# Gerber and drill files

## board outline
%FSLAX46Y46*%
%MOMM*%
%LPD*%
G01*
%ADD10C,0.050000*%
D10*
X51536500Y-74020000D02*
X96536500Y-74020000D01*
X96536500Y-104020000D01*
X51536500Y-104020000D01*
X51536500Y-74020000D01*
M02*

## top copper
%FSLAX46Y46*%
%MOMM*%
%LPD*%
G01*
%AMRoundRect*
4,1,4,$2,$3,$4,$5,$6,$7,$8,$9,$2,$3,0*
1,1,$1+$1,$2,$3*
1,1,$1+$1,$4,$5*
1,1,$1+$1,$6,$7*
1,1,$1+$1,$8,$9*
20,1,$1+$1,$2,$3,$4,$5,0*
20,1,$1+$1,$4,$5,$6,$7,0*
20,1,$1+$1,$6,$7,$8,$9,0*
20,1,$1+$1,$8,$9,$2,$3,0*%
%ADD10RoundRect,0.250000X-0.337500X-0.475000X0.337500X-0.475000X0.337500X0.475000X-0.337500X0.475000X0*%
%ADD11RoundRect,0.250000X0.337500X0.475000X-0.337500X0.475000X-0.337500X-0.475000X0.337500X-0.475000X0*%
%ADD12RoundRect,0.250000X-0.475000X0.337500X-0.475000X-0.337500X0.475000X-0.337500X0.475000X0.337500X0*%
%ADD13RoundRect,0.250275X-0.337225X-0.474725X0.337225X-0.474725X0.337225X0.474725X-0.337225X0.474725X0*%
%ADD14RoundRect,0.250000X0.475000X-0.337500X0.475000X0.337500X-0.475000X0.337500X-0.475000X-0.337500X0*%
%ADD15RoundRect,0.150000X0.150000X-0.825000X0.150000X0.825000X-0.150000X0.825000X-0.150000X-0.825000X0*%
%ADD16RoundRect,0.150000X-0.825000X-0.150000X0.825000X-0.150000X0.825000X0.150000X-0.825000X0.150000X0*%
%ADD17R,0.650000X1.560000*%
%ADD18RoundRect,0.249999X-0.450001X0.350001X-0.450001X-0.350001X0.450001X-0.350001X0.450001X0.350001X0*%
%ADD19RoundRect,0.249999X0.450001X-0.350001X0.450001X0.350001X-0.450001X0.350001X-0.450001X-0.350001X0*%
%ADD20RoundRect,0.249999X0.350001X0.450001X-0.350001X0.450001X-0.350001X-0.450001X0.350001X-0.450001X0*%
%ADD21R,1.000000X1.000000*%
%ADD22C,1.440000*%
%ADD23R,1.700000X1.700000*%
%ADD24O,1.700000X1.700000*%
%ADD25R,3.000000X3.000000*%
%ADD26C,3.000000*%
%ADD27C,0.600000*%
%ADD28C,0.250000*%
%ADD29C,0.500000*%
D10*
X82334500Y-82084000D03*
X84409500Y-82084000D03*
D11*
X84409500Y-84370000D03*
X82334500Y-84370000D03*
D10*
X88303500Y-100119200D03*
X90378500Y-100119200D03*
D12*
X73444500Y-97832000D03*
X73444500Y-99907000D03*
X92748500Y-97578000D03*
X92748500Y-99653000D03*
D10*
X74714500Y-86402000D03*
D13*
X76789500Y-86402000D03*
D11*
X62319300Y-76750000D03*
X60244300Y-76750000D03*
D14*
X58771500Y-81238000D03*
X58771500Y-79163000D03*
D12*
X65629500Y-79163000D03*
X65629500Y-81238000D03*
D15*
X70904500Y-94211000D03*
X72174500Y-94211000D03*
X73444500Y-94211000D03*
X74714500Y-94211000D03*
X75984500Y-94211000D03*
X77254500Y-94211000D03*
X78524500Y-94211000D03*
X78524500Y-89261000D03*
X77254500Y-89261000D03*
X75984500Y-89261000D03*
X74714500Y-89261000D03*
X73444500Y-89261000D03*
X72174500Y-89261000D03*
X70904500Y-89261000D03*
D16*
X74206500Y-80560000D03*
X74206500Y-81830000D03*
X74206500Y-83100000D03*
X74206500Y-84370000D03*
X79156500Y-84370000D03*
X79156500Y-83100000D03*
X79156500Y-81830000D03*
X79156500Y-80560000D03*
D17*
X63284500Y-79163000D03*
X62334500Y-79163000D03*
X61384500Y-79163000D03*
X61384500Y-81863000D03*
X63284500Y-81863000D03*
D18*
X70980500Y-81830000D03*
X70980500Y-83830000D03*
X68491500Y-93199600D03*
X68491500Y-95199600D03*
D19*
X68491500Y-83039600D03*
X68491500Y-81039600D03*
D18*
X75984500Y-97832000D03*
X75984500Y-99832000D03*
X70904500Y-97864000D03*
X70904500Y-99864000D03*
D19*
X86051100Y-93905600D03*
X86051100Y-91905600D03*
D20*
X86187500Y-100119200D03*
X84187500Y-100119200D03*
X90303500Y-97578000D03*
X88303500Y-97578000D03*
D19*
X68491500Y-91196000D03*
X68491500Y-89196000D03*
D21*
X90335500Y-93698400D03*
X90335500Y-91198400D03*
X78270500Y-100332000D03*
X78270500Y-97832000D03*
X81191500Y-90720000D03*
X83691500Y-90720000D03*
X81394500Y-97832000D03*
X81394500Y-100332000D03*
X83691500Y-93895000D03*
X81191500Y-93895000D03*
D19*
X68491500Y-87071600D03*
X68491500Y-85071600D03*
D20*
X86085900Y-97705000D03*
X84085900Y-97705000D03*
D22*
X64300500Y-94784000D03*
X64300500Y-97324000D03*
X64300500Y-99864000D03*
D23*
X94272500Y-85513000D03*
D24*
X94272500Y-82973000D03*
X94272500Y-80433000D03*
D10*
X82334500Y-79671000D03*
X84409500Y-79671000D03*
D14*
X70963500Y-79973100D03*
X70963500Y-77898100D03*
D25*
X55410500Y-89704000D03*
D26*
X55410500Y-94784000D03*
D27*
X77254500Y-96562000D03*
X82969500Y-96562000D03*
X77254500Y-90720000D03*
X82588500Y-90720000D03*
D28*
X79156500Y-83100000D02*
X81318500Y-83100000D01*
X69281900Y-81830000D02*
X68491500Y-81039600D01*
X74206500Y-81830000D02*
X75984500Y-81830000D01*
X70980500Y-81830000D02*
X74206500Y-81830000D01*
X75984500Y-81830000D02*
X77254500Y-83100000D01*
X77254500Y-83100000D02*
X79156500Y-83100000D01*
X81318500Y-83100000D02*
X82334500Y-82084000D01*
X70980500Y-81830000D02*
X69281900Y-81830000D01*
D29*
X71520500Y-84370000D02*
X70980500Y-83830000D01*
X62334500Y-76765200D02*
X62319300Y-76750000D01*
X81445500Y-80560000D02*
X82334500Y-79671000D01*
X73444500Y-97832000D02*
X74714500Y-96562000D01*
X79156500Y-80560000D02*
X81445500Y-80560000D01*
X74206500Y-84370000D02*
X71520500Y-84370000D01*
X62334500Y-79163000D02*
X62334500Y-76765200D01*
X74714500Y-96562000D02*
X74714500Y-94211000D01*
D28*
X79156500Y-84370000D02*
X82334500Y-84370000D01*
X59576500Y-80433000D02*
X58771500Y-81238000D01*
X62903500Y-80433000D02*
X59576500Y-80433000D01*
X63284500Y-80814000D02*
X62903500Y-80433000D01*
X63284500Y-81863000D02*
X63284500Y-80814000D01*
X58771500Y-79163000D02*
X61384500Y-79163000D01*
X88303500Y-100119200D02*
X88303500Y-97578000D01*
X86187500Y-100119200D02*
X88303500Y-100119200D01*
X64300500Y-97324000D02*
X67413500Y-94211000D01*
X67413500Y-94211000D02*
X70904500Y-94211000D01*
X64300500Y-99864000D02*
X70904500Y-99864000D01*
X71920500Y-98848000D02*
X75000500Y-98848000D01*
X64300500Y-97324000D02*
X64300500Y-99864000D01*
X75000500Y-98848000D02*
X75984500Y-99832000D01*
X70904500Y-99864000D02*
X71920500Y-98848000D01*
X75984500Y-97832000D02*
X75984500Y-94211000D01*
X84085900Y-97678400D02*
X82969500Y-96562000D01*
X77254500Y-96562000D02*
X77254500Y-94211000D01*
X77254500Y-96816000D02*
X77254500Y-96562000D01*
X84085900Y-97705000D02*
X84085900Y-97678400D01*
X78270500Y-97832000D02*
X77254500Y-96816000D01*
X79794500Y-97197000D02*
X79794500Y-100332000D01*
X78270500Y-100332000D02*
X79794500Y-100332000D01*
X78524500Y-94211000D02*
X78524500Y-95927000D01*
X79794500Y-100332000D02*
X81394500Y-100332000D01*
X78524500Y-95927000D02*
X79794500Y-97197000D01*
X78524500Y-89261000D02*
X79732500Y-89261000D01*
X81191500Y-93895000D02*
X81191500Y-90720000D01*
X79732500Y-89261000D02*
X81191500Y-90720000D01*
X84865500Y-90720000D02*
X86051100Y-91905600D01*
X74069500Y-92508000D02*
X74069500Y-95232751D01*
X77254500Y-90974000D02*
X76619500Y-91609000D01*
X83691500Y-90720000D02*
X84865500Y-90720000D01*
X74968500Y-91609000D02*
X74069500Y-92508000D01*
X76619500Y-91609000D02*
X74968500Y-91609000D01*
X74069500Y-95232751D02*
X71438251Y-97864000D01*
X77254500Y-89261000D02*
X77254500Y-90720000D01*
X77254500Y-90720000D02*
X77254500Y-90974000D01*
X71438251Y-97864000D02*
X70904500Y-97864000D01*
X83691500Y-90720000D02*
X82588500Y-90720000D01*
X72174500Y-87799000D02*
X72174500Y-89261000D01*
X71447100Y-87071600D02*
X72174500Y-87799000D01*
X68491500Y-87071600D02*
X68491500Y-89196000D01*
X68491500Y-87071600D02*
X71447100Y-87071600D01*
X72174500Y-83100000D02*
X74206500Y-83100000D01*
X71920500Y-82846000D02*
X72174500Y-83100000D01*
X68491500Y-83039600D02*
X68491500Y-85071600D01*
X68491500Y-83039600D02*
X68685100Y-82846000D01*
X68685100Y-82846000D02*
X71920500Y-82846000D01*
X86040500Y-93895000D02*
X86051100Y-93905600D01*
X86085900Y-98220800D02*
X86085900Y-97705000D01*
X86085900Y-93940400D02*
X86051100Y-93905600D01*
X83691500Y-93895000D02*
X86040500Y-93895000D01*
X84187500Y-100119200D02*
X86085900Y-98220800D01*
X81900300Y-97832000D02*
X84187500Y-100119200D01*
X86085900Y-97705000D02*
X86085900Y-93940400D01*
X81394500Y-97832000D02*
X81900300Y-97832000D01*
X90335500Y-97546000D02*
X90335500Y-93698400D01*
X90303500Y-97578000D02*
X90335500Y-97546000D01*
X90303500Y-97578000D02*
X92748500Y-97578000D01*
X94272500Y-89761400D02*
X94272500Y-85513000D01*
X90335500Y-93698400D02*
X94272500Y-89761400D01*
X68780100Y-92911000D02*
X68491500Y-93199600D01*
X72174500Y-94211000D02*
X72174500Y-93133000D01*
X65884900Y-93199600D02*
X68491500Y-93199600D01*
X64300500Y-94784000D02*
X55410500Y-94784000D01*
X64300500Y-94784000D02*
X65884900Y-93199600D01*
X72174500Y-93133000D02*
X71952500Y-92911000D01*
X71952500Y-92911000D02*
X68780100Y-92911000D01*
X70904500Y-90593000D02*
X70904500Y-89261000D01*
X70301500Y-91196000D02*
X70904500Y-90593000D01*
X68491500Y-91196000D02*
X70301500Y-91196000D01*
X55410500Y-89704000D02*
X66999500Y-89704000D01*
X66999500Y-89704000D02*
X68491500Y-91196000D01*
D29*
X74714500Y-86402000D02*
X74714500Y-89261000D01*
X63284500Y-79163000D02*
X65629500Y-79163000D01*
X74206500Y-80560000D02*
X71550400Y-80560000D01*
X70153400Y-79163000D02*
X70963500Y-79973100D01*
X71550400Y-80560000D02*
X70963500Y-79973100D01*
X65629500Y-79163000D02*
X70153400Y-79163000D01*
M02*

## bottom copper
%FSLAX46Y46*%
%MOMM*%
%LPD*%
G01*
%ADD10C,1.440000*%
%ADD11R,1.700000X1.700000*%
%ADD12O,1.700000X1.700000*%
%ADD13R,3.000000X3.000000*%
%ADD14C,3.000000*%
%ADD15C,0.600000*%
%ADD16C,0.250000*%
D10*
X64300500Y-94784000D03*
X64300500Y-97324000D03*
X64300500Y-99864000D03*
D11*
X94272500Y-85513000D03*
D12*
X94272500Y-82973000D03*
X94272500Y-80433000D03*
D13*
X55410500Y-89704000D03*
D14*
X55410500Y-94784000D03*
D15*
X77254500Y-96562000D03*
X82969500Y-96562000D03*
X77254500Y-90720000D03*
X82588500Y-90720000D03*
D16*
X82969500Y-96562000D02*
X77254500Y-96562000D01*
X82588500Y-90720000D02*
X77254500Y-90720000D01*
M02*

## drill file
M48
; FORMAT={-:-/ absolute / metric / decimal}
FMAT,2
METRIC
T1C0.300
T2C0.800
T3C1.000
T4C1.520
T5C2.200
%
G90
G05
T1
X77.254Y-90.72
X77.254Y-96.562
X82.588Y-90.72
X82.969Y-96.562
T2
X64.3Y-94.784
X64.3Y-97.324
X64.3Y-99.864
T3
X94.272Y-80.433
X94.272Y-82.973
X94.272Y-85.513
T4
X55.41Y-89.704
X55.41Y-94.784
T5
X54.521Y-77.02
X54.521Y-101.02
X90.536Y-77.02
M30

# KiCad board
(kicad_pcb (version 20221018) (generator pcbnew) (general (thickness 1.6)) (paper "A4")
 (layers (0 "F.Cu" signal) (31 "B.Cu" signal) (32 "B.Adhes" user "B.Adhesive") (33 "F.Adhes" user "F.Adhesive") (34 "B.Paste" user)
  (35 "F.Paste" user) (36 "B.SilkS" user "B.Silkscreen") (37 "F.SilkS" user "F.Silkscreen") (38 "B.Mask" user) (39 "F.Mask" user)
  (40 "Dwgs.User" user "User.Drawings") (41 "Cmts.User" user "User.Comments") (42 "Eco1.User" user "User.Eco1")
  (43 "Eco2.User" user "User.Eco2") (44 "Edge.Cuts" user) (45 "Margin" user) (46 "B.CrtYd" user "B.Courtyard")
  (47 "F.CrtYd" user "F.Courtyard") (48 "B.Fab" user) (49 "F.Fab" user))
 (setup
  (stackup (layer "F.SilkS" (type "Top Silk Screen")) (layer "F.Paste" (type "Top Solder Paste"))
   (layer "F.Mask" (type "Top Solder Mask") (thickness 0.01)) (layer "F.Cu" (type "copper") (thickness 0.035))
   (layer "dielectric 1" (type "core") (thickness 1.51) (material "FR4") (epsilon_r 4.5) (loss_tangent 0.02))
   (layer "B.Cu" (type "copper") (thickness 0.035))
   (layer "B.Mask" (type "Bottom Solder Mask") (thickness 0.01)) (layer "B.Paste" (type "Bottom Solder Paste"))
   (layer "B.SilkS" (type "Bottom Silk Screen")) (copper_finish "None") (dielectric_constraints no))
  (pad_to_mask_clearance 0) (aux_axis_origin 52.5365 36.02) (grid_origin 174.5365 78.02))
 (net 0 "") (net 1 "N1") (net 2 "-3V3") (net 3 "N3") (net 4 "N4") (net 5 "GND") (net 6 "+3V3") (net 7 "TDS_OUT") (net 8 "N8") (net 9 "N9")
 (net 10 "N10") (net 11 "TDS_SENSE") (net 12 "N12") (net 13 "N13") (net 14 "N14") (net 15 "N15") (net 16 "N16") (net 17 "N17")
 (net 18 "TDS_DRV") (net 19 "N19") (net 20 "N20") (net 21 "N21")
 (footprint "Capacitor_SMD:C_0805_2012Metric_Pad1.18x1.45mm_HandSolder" (layer "F.Cu") (at 83.372 82.084)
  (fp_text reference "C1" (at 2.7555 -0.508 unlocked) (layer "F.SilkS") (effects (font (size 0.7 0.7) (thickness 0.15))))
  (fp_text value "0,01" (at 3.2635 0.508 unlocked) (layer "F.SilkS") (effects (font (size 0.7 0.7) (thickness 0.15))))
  (pad "1" smd roundrect (at -1.0375 0) (size 1.175 1.45) (layers "F.Cu" "F.Paste" "F.Mask") (roundrect_rratio 0.2127659574) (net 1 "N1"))
  (pad "2" smd roundrect (at 1.0375 0) (size 1.175 1.45) (layers "F.Cu" "F.Paste" "F.Mask") (roundrect_rratio 0.2127659574) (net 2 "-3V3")))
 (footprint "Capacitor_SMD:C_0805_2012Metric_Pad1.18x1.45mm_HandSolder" (layer "F.Cu") (at 83.372 84.37 180)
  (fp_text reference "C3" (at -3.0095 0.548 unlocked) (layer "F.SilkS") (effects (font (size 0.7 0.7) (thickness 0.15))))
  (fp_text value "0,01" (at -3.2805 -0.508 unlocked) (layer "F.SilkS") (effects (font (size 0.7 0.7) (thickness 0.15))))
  (pad "1" smd roundrect (at -1.0375 0 180) (size 1.175 1.45) (layers "F.Cu" "F.Paste" "F.Mask") (roundrect_rratio 0.2127659574)
   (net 2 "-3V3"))
  (pad "2" smd roundrect (at 1.0375 0 180) (size 1.175 1.45) (layers "F.Cu" "F.Paste" "F.Mask") (roundrect_rratio 0.2127659574) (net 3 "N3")))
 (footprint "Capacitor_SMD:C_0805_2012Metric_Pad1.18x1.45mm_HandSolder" (layer "F.Cu") (at 89.341 100.1192)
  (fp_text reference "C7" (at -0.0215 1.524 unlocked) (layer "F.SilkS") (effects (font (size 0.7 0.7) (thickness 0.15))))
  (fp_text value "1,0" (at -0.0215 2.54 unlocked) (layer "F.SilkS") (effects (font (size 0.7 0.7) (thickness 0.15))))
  (pad "1" smd roundrect (at -1.0375 0) (size 1.175 1.45) (layers "F.Cu" "F.Paste" "F.Mask") (roundrect_rratio 0.2127659574) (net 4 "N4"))
  (pad "2" smd roundrect (at 1.0375 0) (size 1.175 1.45) (layers "F.Cu" "F.Paste" "F.Mask") (roundrect_rratio 0.2127659574) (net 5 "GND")))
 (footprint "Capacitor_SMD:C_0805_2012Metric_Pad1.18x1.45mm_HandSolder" (layer "F.Cu") (at 73.4445 98.8695 -90)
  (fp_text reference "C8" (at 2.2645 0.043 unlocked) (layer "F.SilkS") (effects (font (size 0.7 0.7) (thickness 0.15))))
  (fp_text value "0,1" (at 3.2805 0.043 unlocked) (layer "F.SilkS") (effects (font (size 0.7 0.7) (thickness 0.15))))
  (pad "1" smd roundrect (at -1.0375 0 270) (size 1.175 1.45) (layers "F.Cu" "F.Paste" "F.Mask") (roundrect_rratio 0.2127659574)
   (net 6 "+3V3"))
  (pad "2" smd roundrect (at 1.0375 0 270) (size 1.175 1.45) (layers "F.Cu" "F.Paste" "F.Mask") (roundrect_rratio 0.2127659574)
   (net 5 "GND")))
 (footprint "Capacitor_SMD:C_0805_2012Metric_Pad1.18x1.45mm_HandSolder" (layer "F.Cu") (at 92.7485 98.6155 -90)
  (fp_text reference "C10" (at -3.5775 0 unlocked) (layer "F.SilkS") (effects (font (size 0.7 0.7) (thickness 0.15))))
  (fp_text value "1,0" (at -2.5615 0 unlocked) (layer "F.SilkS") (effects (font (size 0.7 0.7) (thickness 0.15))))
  (pad "1" smd roundrect (at -1.0375 0 270) (size 1.175 1.45) (layers "F.Cu" "F.Paste" "F.Mask") (roundrect_rratio 0.2127659574)
   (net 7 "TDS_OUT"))
  (pad "2" smd roundrect (at 1.0375 0 270) (size 1.175 1.45) (layers "F.Cu" "F.Paste" "F.Mask") (roundrect_rratio 0.2127659574)
   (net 5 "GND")))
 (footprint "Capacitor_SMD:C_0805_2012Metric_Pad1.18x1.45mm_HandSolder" (layer "F.Cu") (at 75.752 86.402)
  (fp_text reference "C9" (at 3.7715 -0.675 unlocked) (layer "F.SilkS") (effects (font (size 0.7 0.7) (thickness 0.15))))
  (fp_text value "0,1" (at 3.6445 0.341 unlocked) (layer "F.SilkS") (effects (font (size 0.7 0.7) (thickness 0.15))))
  (pad "1" smd roundrect (at -1.0375 0) (size 1.175 1.45) (layers "F.Cu" "F.Paste" "F.Mask") (roundrect_rratio 0.2127659574) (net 2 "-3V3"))
  (pad "2" smd roundrect (at 1.0375 0) (size 1.175 1.45) (layers "F.Cu" "F.Paste" "F.Mask") (roundrect_rratio 0.213) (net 5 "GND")))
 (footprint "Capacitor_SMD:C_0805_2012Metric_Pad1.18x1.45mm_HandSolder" (layer "F.Cu") (at 61.2818 76.75 180)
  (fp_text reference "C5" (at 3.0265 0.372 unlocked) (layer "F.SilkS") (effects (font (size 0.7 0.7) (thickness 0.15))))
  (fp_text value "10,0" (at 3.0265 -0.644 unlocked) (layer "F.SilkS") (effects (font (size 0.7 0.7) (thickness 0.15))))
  (pad "1" smd roundrect (at -1.0375 0 180) (size 1.175 1.45) (layers "F.Cu" "F.Paste" "F.Mask") (roundrect_rratio 0.2127659574)
   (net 6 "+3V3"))
  (pad "2" smd roundrect (at 1.0375 0 180) (size 1.175 1.45) (layers "F.Cu" "F.Paste" "F.Mask") (roundrect_rratio 0.2127659574)
   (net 5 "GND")))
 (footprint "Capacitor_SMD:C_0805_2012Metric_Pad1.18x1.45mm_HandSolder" (layer "F.Cu") (at 58.7715 80.2005 90)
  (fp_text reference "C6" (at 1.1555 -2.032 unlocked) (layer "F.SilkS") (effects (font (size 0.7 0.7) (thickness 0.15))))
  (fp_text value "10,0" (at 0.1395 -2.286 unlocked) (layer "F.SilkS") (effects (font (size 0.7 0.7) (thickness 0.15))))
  (pad "1" smd roundrect (at -1.0375 0 90) (size 1.175 1.45) (layers "F.Cu" "F.Paste" "F.Mask") (roundrect_rratio 0.2127659574) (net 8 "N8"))
  (pad "2" smd roundrect (at 1.0375 0 90) (size 1.175 1.45) (layers "F.Cu" "F.Paste" "F.Mask") (roundrect_rratio 0.2127659574) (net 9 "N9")))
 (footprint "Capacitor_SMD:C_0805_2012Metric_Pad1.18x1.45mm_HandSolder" (layer "F.Cu") (at 65.6295 80.2005 -90)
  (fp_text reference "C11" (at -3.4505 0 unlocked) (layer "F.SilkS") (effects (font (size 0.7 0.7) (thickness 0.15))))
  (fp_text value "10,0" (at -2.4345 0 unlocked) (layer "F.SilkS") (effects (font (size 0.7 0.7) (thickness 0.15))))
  (pad "1" smd roundrect (at -1.0375 0 270) (size 1.175 1.45) (layers "F.Cu" "F.Paste" "F.Mask") (roundrect_rratio 0.2127659574)
   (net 2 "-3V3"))
  (pad "2" smd roundrect (at 1.0375 0 270) (size 1.175 1.45) (layers "F.Cu" "F.Paste" "F.Mask") (roundrect_rratio 0.2127659574)
   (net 5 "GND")))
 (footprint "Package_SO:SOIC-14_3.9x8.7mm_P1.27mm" (layer "F.Cu") (at 74.7145 91.736 90)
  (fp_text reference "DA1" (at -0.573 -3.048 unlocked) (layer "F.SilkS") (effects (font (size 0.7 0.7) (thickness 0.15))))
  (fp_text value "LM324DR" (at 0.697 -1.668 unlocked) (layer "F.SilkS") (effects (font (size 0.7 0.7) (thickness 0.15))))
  (pad "1" smd roundrect (at -2.475 -3.81 90) (size 1.95 0.6) (layers "F.Cu" "F.Paste" "F.Mask") (roundrect_rratio 0.25) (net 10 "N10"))
  (pad "2" smd roundrect (at -2.475 -2.54 90) (size 1.95 0.6) (layers "F.Cu" "F.Paste" "F.Mask") (roundrect_rratio 0.25)
   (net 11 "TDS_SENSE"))
  (pad "3" smd roundrect (at -2.475 -1.27 90) (size 1.95 0.6) (layers "F.Cu" "F.Paste" "F.Mask") (roundrect_rratio 0.25) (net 5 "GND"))
  (pad "4" smd roundrect (at -2.475 0 90) (size 1.95 0.6) (layers "F.Cu" "F.Paste" "F.Mask") (roundrect_rratio 0.25) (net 6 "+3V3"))
  (pad "5" smd roundrect (at -2.475 1.27 90) (size 1.95 0.6) (layers "F.Cu" "F.Paste" "F.Mask") (roundrect_rratio 0.25) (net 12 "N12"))
  (pad "6" smd roundrect (at -2.475 2.54 90) (size 1.95 0.6) (layers "F.Cu" "F.Paste" "F.Mask") (roundrect_rratio 0.25) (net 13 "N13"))
  (pad "7" smd roundrect (at -2.475 3.81 90) (size 1.95 0.6) (layers "F.Cu" "F.Paste" "F.Mask") (roundrect_rratio 0.25) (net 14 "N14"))
  (pad "8" smd roundrect (at 2.475 3.81 90) (size 1.95 0.6) (layers "F.Cu" "F.Paste" "F.Mask") (roundrect_rratio 0.25) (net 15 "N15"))
  (pad "9" smd roundrect (at 2.475 2.54 90) (size 1.95 0.6) (layers "F.Cu" "F.Paste" "F.Mask") (roundrect_rratio 0.25) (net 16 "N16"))
  (pad "10" smd roundrect (at 2.475 1.27 90) (size 1.95 0.6) (layers "F.Cu" "F.Paste" "F.Mask") (roundrect_rratio 0.25) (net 5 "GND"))
  (pad "11" smd roundrect (at 2.475 0 90) (size 1.95 0.6) (layers "F.Cu" "F.Paste" "F.Mask") (roundrect_rratio 0.25) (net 2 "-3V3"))
  (pad "12" smd roundrect (at 2.475 -1.27 90) (size 1.95 0.6) (layers "F.Cu" "F.Paste" "F.Mask") (roundrect_rratio 0.25) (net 5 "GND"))
  (pad "13" smd roundrect (at 2.475 -2.54 90) (size 1.95 0.6) (layers "F.Cu" "F.Paste" "F.Mask") (roundrect_rratio 0.25) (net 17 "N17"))
  (pad "14" smd roundrect (at 2.475 -3.81 90) (size 1.95 0.6) (layers "F.Cu" "F.Paste" "F.Mask") (roundrect_rratio 0.25) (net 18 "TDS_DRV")))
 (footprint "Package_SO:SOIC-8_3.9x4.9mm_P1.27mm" (layer "F.Cu") (at 76.6815 82.465)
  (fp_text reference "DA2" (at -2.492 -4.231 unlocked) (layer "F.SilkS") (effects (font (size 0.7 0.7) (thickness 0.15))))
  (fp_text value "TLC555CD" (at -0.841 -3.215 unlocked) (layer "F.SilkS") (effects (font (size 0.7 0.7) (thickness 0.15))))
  (pad "1" smd roundrect (at -2.475 -1.905) (size 1.95 0.6) (layers "F.Cu" "F.Paste" "F.Mask") (roundrect_rratio 0.25) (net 2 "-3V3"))
  (pad "2" smd roundrect (at -2.475 -0.635) (size 1.95 0.6) (layers "F.Cu" "F.Paste" "F.Mask") (roundrect_rratio 0.25) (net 1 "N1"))
  (pad "3" smd roundrect (at -2.475 0.635) (size 1.95 0.6) (layers "F.Cu" "F.Paste" "F.Mask") (roundrect_rratio 0.25) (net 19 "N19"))
  (pad "4" smd roundrect (at -2.475 1.905) (size 1.95 0.6) (layers "F.Cu" "F.Paste" "F.Mask") (roundrect_rratio 0.25) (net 6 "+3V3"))
  (pad "5" smd roundrect (at 2.475 1.905) (size 1.95 0.6) (layers "F.Cu" "F.Paste" "F.Mask") (roundrect_rratio 0.25) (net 3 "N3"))
  (pad "6" smd roundrect (at 2.475 0.635) (size 1.95 0.6) (layers "F.Cu" "F.Paste" "F.Mask") (roundrect_rratio 0.25) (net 1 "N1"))
  (pad "7" smd roundrect (at 2.475 -0.635) (size 1.95 0.6) (layers "F.Cu" "F.Paste" "F.Mask") (roundrect_rratio 0.25) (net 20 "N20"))
  (pad "8" smd roundrect (at 2.475 -1.905) (size 1.95 0.6) (layers "F.Cu" "F.Paste" "F.Mask") (roundrect_rratio 0.25) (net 6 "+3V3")))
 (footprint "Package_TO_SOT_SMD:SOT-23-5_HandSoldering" (layer "F.Cu") (at 62.3345 80.513 -90)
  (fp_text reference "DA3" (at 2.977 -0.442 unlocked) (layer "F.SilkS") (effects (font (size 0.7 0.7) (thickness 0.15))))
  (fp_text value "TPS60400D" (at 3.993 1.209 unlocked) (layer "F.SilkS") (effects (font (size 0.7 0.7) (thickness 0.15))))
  (pad "1" smd rect (at -1.35 -0.95 270) (size 1.56 0.65) (layers "F.Cu" "F.Paste" "F.Mask") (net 2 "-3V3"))
  (pad "2" smd rect (at -1.35 0 270) (size 1.56 0.65) (layers "F.Cu" "F.Paste" "F.Mask") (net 6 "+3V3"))
  (pad "3" smd rect (at -1.35 0.95 270) (size 1.56 0.65) (layers "F.Cu" "F.Paste" "F.Mask") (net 9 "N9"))
  (pad "4" smd rect (at 1.35 0.95 270) (size 1.56 0.65) (layers "F.Cu" "F.Paste" "F.Mask") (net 5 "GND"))
  (pad "5" smd rect (at 1.35 -0.95 270) (size 1.56 0.65) (layers "F.Cu" "F.Paste" "F.Mask") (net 8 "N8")))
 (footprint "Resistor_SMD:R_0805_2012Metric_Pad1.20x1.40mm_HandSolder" (layer "F.Cu") (at 70.9805 82.83 -90)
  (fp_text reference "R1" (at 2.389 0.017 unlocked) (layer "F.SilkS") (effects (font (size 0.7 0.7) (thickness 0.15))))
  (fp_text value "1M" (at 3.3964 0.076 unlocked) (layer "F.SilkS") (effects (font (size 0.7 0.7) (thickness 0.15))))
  (pad "1" smd roundrect (at -1 0 270) (size 1.2 1.4) (layers "F.Cu" "F.Paste" "F.Mask") (roundrect_rratio 0.2083325) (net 1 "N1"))
  (pad "2" smd roundrect (at 1 0 270) (size 1.2 1.4) (layers "F.Cu" "F.Paste" "F.Mask") (roundrect_rratio 0.2083325) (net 6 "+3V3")))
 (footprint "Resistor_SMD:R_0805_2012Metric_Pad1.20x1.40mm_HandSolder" (layer "F.Cu") (at 68.4915 94.1996 -90)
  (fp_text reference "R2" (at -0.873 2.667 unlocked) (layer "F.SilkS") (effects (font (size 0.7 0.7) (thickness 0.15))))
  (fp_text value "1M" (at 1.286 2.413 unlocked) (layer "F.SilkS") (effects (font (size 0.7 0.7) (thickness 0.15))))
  (pad "1" smd roundrect (at -1 0 270) (size 1.2 1.4) (layers "F.Cu" "F.Paste" "F.Mask") (roundrect_rratio 0.2083325) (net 11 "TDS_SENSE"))
  (pad "2" smd roundrect (at 1 0 270) (size 1.2 1.4) (layers "F.Cu" "F.Paste" "F.Mask") (roundrect_rratio 0.2083325) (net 5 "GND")))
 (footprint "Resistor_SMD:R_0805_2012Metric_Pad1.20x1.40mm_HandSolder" (layer "F.Cu") (at 68.4915 82.0396 90)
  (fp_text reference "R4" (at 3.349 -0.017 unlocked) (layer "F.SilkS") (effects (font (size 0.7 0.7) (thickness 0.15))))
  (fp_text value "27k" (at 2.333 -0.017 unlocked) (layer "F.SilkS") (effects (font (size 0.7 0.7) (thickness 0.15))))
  (pad "1" smd roundrect (at -1 0 90) (size 1.2 1.4) (layers "F.Cu" "F.Paste" "F.Mask") (roundrect_rratio 0.2083325) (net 19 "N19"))
  (pad "2" smd roundrect (at 1 0 90) (size 1.2 1.4) (layers "F.Cu" "F.Paste" "F.Mask") (roundrect_rratio 0.2083325) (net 1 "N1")))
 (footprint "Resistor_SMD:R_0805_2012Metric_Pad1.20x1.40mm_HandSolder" (layer "F.Cu") (at 75.9845 98.832 -90)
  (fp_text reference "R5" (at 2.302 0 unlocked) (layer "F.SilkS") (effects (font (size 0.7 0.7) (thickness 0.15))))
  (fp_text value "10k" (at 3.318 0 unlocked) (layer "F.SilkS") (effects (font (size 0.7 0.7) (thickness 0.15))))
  (pad "1" smd roundrect (at -1 0 270) (size 1.2 1.4) (layers "F.Cu" "F.Paste" "F.Mask") (roundrect_rratio 0.2083325) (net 12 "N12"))
  (pad "2" smd roundrect (at 1 0 270) (size 1.2 1.4) (layers "F.Cu" "F.Paste" "F.Mask") (roundrect_rratio 0.2083325) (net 10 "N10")))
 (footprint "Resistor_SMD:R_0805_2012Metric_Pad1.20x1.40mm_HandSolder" (layer "F.Cu") (at 70.9045 98.864 -90)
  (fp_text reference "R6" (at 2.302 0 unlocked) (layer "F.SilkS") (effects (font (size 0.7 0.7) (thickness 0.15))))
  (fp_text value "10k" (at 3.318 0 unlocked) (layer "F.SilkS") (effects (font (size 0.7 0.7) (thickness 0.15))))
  (pad "1" smd roundrect (at -1 0 270) (size 1.2 1.4) (layers "F.Cu" "F.Paste" "F.Mask") (roundrect_rratio 0.2083325) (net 16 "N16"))
  (pad "2" smd roundrect (at 1 0 270) (size 1.2 1.4) (layers "F.Cu" "F.Paste" "F.Mask") (roundrect_rratio 0.2083325) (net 10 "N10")))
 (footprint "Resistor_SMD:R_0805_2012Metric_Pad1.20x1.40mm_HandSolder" (layer "F.Cu") (at 86.0511 92.9056 90)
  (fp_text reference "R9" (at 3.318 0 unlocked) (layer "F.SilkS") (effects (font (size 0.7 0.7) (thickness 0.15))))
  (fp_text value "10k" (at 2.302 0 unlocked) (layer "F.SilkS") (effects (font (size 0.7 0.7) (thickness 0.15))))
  (pad "1" smd roundrect (at -1 0 90) (size 1.2 1.4) (layers "F.Cu" "F.Paste" "F.Mask") (roundrect_rratio 0.2083325) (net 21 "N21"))
  (pad "2" smd roundrect (at 1 0 90) (size 1.2 1.4) (layers "F.Cu" "F.Paste" "F.Mask") (roundrect_rratio 0.2083325) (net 16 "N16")))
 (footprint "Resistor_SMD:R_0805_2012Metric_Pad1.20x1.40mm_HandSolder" (layer "F.Cu") (at 85.1875 100.1192 180)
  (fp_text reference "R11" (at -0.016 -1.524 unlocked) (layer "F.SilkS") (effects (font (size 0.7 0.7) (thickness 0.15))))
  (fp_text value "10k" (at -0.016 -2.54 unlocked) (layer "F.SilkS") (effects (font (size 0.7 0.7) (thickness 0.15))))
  (pad "1" smd roundrect (at -1 0 180) (size 1.2 1.4) (layers "F.Cu" "F.Paste" "F.Mask") (roundrect_rratio 0.2083325) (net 4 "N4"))
  (pad "2" smd roundrect (at 1 0 180) (size 1.2 1.4) (layers "F.Cu" "F.Paste" "F.Mask") (roundrect_rratio 0.2083325) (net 21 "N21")))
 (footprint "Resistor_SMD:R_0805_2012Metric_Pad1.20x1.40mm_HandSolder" (layer "F.Cu") (at 89.3035 97.578 180)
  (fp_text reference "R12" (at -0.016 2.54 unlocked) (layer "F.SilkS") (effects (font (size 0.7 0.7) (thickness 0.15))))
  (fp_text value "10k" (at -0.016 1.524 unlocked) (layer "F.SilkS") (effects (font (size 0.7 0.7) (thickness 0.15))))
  (pad "1" smd roundrect (at -1 0 180) (size 1.2 1.4) (layers "F.Cu" "F.Paste" "F.Mask") (roundrect_rratio 0.2083325) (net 7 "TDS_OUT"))
  (pad "2" smd roundrect (at 1 0 180) (size 1.2 1.4) (layers "F.Cu" "F.Paste" "F.Mask") (roundrect_rratio 0.2083325) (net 4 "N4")))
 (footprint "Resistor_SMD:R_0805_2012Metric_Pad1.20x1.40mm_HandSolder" (layer "F.Cu") (at 68.4915 90.196 90)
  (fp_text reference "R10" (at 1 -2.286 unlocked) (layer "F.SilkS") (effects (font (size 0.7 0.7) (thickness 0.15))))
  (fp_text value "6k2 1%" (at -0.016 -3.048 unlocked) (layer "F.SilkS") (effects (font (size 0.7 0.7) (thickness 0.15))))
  (pad "1" smd roundrect (at -1 0 90) (size 1.2 1.4) (layers "F.Cu" "F.Paste" "F.Mask") (roundrect_rratio 0.2083325) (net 18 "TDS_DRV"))
  (pad "2" smd roundrect (at 1 0 90) (size 1.2 1.4) (layers "F.Cu" "F.Paste" "F.Mask") (roundrect_rratio 0.2083325) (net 17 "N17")))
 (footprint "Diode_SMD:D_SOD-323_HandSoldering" (layer "F.Cu") (at 90.3355 92.4484 90)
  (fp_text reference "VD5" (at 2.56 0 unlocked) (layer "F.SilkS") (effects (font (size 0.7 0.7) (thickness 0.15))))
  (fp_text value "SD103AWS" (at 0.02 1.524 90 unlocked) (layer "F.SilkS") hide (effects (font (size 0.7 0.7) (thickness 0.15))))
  (pad "1" smd rect (at -1.25 0 90) (size 1 1) (layers "F.Cu" "F.Paste" "F.Mask") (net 7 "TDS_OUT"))
  (pad "2" smd rect (at 1.25 0 90) (size 1 1) (layers "F.Cu" "F.Paste" "F.Mask") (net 5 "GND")))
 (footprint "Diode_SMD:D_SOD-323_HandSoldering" (layer "F.Cu") (at 78.2705 99.082 90)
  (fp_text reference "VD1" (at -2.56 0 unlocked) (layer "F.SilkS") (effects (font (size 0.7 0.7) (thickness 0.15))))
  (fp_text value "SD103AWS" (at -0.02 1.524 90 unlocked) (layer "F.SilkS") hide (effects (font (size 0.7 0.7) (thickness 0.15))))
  (pad "1" smd rect (at -1.25 0 90) (size 1 1) (layers "F.Cu" "F.Paste" "F.Mask") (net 14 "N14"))
  (pad "2" smd rect (at 1.25 0 90) (size 1 1) (layers "F.Cu" "F.Paste" "F.Mask") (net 13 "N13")))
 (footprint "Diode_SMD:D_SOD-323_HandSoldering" (layer "F.Cu") (at 82.4415 90.72)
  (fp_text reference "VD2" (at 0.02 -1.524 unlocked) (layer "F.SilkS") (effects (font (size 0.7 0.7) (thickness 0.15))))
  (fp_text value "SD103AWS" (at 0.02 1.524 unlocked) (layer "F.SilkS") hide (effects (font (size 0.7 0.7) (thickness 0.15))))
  (pad "1" smd rect (at -1.25 0) (size 1 1) (layers "F.Cu" "F.Paste" "F.Mask") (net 15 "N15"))
  (pad "2" smd rect (at 1.25 0) (size 1 1) (layers "F.Cu" "F.Paste" "F.Mask") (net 16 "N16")))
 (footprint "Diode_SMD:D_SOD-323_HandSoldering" (layer "F.Cu") (at 81.3945 99.082 -90)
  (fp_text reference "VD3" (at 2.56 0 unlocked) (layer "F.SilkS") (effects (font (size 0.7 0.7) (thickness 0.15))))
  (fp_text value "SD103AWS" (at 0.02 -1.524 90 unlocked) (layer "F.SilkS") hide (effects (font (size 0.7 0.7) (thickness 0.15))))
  (pad "1" smd rect (at -1.25 0 270) (size 1 1) (layers "F.Cu" "F.Paste" "F.Mask") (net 21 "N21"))
  (pad "2" smd rect (at 1.25 0 270) (size 1 1) (layers "F.Cu" "F.Paste" "F.Mask") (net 14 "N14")))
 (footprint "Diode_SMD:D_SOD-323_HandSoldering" (layer "F.Cu") (at 82.4415 93.895 180)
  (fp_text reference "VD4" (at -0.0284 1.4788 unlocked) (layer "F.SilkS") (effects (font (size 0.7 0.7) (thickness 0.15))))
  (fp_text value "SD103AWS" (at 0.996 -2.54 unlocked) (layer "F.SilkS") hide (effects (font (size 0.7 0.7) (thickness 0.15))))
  (pad "1" smd rect (at -1.25 0 180) (size 1 1) (layers "F.Cu" "F.Paste" "F.Mask") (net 21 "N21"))
  (pad "2" smd rect (at 1.25 0 180) (size 1 1) (layers "F.Cu" "F.Paste" "F.Mask") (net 15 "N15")))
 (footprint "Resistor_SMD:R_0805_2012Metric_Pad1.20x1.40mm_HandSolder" (layer "F.Cu") (at 68.4915 86.0716 90)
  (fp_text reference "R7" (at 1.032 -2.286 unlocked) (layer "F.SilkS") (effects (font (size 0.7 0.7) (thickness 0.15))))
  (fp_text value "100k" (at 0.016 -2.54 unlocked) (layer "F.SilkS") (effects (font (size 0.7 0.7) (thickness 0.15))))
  (pad "1" smd roundrect (at -1 0 90) (size 1.2 1.4) (layers "F.Cu" "F.Paste" "F.Mask") (roundrect_rratio 0.2083325) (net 17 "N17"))
  (pad "2" smd roundrect (at 1 0 90) (size 1.2 1.4) (layers "F.Cu" "F.Paste" "F.Mask") (roundrect_rratio 0.2083325) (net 19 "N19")))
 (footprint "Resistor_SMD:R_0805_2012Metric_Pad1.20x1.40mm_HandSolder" (layer "F.Cu") (at 85.0859 97.705 180)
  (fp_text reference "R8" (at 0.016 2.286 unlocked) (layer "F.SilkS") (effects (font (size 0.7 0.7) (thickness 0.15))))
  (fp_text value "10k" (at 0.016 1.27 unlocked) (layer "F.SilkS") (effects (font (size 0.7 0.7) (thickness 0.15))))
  (pad "1" smd roundrect (at -1 0 180) (size 1.2 1.4) (layers "F.Cu" "F.Paste" "F.Mask") (roundrect_rratio 0.2083325) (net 21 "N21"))
  (pad "2" smd roundrect (at 1 0 180) (size 1.2 1.4) (layers "F.Cu" "F.Paste" "F.Mask") (roundrect_rratio 0.2083325) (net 13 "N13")))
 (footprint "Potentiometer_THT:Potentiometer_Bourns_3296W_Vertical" (layer "F.Cu") (at 64.3005 94.784 90)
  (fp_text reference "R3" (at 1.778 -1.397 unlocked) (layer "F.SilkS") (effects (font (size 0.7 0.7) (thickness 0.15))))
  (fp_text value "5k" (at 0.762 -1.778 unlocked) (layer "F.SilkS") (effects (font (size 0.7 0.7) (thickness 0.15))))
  (pad "1" thru_hole circle (at 0 0 90) (size 1.44 1.44) (drill 0.8) (layers "*.Cu" "*.Mask") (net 11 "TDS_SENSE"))
  (pad "2" thru_hole circle (at -2.54 0 90) (size 1.44 1.44) (drill 0.8) (layers "*.Cu" "*.Mask") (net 10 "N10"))
  (pad "3" thru_hole circle (at -5.08 0 90) (size 1.44 1.44) (drill 0.8) (layers "*.Cu" "*.Mask") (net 10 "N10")))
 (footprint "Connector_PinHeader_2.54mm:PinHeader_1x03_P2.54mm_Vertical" (layer "F.Cu") (at 94.2725 85.513 180)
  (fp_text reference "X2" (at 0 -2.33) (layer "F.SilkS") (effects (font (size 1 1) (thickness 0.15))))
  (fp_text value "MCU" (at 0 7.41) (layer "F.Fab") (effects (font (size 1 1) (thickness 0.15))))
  (pad "1" thru_hole rect (at 0 0 180) (size 1.7 1.7) (drill 1) (layers "*.Cu" "*.Mask") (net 7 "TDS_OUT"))
  (pad "2" thru_hole oval (at 0 2.54 180) (size 1.7 1.7) (drill 1) (layers "*.Cu" "*.Mask") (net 6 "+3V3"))
  (pad "3" thru_hole oval (at 0 5.08 180) (size 1.7 1.7) (drill 1) (layers "*.Cu" "*.Mask") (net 5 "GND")))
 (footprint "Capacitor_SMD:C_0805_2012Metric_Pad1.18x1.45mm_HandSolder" (layer "F.Cu") (at 83.372 79.671)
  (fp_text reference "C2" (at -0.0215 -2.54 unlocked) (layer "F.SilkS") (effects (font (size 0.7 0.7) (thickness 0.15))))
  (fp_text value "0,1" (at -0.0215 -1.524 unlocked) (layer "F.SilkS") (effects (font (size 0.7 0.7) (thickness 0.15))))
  (pad "1" smd roundrect (at -1.0375 0) (size 1.175 1.45) (layers "F.Cu" "F.Paste" "F.Mask") (roundrect_rratio 0.2127659574) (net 6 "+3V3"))
  (pad "2" smd roundrect (at 1.0375 0) (size 1.175 1.45) (layers "F.Cu" "F.Paste" "F.Mask") (roundrect_rratio 0.2127659574) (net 5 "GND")))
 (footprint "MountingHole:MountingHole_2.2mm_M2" (layer "F.Cu") (at 54.5215 77.02)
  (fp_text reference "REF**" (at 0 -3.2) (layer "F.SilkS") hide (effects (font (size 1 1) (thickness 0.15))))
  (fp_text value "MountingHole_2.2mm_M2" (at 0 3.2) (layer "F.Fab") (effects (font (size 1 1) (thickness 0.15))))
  (pad "" np_thru_hole circle (at 0 0) (size 2.2 2.2) (drill 2.2) (layers "*.Cu" "*.Mask")))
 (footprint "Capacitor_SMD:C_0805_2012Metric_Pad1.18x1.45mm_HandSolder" (layer "F.Cu") (at 70.9635 78.9356 90)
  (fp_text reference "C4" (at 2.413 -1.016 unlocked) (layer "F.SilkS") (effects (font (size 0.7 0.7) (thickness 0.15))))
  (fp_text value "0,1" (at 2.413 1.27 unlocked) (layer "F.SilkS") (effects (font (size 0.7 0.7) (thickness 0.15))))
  (pad "1" smd roundrect (at -1.0375 0 90) (size 1.175 1.45) (layers "F.Cu" "F.Paste" "F.Mask") (roundrect_rratio 0.2127659574)
   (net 2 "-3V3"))
  (pad "2" smd roundrect (at 1.0375 0 90) (size 1.175 1.45) (layers "F.Cu" "F.Paste" "F.Mask") (roundrect_rratio 0.2127659574) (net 5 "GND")))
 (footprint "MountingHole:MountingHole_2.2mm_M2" (layer "F.Cu") (at 90.5365 77.02)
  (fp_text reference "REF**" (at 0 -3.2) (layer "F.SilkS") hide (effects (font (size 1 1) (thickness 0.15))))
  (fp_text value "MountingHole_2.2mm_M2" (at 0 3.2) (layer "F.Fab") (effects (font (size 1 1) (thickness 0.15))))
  (pad "" np_thru_hole circle (at 0 0) (size 2.2 2.2) (drill 2.2) (layers "*.Cu" "*.Mask")))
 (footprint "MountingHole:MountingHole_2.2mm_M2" (layer "F.Cu") (at 54.5215 101.02)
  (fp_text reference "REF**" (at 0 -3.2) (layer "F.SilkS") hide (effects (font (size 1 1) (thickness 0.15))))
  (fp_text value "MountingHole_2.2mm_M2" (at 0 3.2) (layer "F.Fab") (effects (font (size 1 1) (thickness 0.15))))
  (pad "" np_thru_hole circle (at 0 0) (size 2.2 2.2) (drill 2.2) (layers "*.Cu" "*.Mask")))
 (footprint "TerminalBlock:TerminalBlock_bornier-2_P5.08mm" (layer "F.Cu") (at 55.4105 89.704 -90)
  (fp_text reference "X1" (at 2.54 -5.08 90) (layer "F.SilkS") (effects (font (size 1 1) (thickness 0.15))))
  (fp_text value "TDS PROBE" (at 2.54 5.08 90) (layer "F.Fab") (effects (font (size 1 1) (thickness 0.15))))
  (pad "1" thru_hole rect (at 0 0 270) (size 3 3) (drill 1.52) (layers "*.Cu" "*.Mask") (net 18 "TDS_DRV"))
  (pad "2" thru_hole circle (at 5.08 0 270) (size 3 3) (drill 1.52) (layers "*.Cu" "*.Mask") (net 11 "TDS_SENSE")))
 (gr_rect (start 51.5365 74.02) (end 96.5365 104.02) (stroke (width 0.05) (type default)) (fill none) (layer "Edge.Cuts"))
 (segment (start 79.1565 83.1) (end 81.3185 83.1) (width 0.25) (layer "F.Cu") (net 1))
 (segment (start 69.2819 81.83) (end 68.4915 81.0396) (width 0.25) (layer "F.Cu") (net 1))
 (segment (start 74.2065 81.83) (end 75.9845 81.83) (width 0.25) (layer "F.Cu") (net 1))
 (segment (start 70.9805 81.83) (end 74.2065 81.83) (width 0.25) (layer "F.Cu") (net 1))
 (segment (start 75.9845 81.83) (end 77.2545 83.1) (width 0.25) (layer "F.Cu") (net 1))
 (segment (start 77.2545 83.1) (end 79.1565 83.1) (width 0.25) (layer "F.Cu") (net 1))
 (segment (start 81.3185 83.1) (end 82.3345 82.084) (width 0.25) (layer "F.Cu") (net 1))
 (segment (start 70.9805 81.83) (end 69.2819 81.83) (width 0.25) (layer "F.Cu") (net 1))
 (segment (start 71.5205 84.37) (end 70.9805 83.83) (width 0.5) (layer "F.Cu") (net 6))
 (segment (start 62.3345 76.7652) (end 62.3193 76.75) (width 0.5) (layer "F.Cu") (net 6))
 (segment (start 81.4455 80.56) (end 82.3345 79.671) (width 0.5) (layer "F.Cu") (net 6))
 (segment (start 73.4445 97.832) (end 74.7145 96.562) (width 0.5) (layer "F.Cu") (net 6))
 (segment (start 79.1565 80.56) (end 81.4455 80.56) (width 0.5) (layer "F.Cu") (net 6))
 (segment (start 74.2065 84.37) (end 71.5205 84.37) (width 0.5) (layer "F.Cu") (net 6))
 (segment (start 62.3345 79.163) (end 62.3345 76.7652) (width 0.5) (layer "F.Cu") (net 6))
 (segment (start 74.7145 96.562) (end 74.7145 94.211) (width 0.5) (layer "F.Cu") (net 6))
 (segment (start 79.1565 84.37) (end 82.3345 84.37) (width 0.25) (layer "F.Cu") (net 3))
 (segment (start 59.5765 80.433) (end 58.7715 81.238) (width 0.25) (layer "F.Cu") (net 8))
 (segment (start 62.9035 80.433) (end 59.5765 80.433) (width 0.25) (layer "F.Cu") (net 8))
 (segment (start 63.2845 80.814) (end 62.9035 80.433) (width 0.25) (layer "F.Cu") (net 8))
 (segment (start 63.2845 81.863) (end 63.2845 80.814) (width 0.25) (layer "F.Cu") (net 8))
 (segment (start 58.7715 79.163) (end 61.3845 79.163) (width 0.25) (layer "F.Cu") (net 9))
 (segment (start 88.3035 100.1192) (end 88.3035 97.578) (width 0.25) (layer "F.Cu") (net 4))
 (segment (start 86.1875 100.1192) (end 88.3035 100.1192) (width 0.25) (layer "F.Cu") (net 4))
 (segment (start 64.3005 97.324) (end 67.4135 94.211) (width 0.25) (layer "F.Cu") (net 10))
 (segment (start 67.4135 94.211) (end 70.9045 94.211) (width 0.25) (layer "F.Cu") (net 10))
 (segment (start 64.3005 99.864) (end 70.9045 99.864) (width 0.25) (layer "F.Cu") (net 10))
 (segment (start 71.9205 98.848) (end 75.0005 98.848) (width 0.25) (layer "F.Cu") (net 10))
 (segment (start 64.3005 97.324) (end 64.3005 99.864) (width 0.25) (layer "F.Cu") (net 10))
 (segment (start 75.0005 98.848) (end 75.9845 99.832) (width 0.25) (layer "F.Cu") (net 10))
 (segment (start 70.9045 99.864) (end 71.9205 98.848) (width 0.25) (layer "F.Cu") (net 10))
 (segment (start 75.9845 97.832) (end 75.9845 94.211) (width 0.25) (layer "F.Cu") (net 12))
 (segment (start 84.0859 97.6784) (end 82.9695 96.562) (width 0.25) (layer "F.Cu") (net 13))
 (segment (start 77.2545 96.562) (end 77.2545 94.211) (width 0.25) (layer "F.Cu") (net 13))
 (segment (start 77.2545 96.816) (end 77.2545 96.562) (width 0.25) (layer "F.Cu") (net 13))
 (segment (start 84.0859 97.705) (end 84.0859 97.6784) (width 0.25) (layer "F.Cu") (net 13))
 (segment (start 78.2705 97.832) (end 77.2545 96.816) (width 0.25) (layer "F.Cu") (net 13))
 (via (at 77.2545 96.562) (size 0.6) (drill 0.3) (layers "F.Cu" "B.Cu") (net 13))
 (via (at 82.9695 96.562) (size 0.6) (drill 0.3) (layers "F.Cu" "B.Cu") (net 13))
 (segment (start 82.9695 96.562) (end 77.2545 96.562) (width 0.25) (layer "B.Cu") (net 13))
 (segment (start 79.7945 97.197) (end 79.7945 100.332) (width 0.25) (layer "F.Cu") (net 14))
 (segment (start 78.2705 100.332) (end 79.7945 100.332) (width 0.25) (layer "F.Cu") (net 14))
 (segment (start 78.5245 94.211) (end 78.5245 95.927) (width 0.25) (layer "F.Cu") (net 14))
 (segment (start 79.7945 100.332) (end 81.3945 100.332) (width 0.25) (layer "F.Cu") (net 14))
 (segment (start 78.5245 95.927) (end 79.7945 97.197) (width 0.25) (layer "F.Cu") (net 14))
 (segment (start 78.5245 89.261) (end 79.7325 89.261) (width 0.25) (layer "F.Cu") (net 15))
 (segment (start 81.1915 93.895) (end 81.1915 90.72) (width 0.25) (layer "F.Cu") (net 15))
 (segment (start 79.7325 89.261) (end 81.1915 90.72) (width 0.25) (layer "F.Cu") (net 15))
 (segment (start 84.8655 90.72) (end 86.0511 91.9056) (width 0.25) (layer "F.Cu") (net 16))
 (segment (start 74.0695 92.508) (end 74.0695 95.232751) (width 0.25) (layer "F.Cu") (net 16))
 (segment (start 77.2545 90.974) (end 76.6195 91.609) (width 0.25) (layer "F.Cu") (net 16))
 (segment (start 83.6915 90.72) (end 84.8655 90.72) (width 0.25) (layer "F.Cu") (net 16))
 (segment (start 74.9685 91.609) (end 74.0695 92.508) (width 0.25) (layer "F.Cu") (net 16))
 (segment (start 76.6195 91.609) (end 74.9685 91.609) (width 0.25) (layer "F.Cu") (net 16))
 (segment (start 74.0695 95.232751) (end 71.438251 97.864) (width 0.25) (layer "F.Cu") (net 16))
 (segment (start 77.2545 89.261) (end 77.2545 90.72) (width 0.25) (layer "F.Cu") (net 16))
 (segment (start 77.2545 90.72) (end 77.2545 90.974) (width 0.25) (layer "F.Cu") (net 16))
 (segment (start 71.438251 97.864) (end 70.9045 97.864) (width 0.25) (layer "F.Cu") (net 16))
 (segment (start 83.6915 90.72) (end 82.5885 90.72) (width 0.25) (layer "F.Cu") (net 16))
 (via (at 77.2545 90.72) (size 0.6) (drill 0.3) (layers "F.Cu" "B.Cu") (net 16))
 (via (at 82.5885 90.72) (size 0.6) (drill 0.3) (layers "F.Cu" "B.Cu") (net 16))
 (segment (start 82.5885 90.72) (end 77.2545 90.72) (width 0.25) (layer "B.Cu") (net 16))
 (segment (start 72.1745 87.799) (end 72.1745 89.261) (width 0.25) (layer "F.Cu") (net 17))
 (segment (start 71.4471 87.0716) (end 72.1745 87.799) (width 0.25) (layer "F.Cu") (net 17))
 (segment (start 68.4915 87.0716) (end 68.4915 89.196) (width 0.25) (layer "F.Cu") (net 17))
 (segment (start 68.4915 87.0716) (end 71.4471 87.0716) (width 0.25) (layer "F.Cu") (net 17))
 (segment (start 72.1745 83.1) (end 74.2065 83.1) (width 0.25) (layer "F.Cu") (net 19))
 (segment (start 71.9205 82.846) (end 72.1745 83.1) (width 0.25) (layer "F.Cu") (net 19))
 (segment (start 68.4915 83.0396) (end 68.4915 85.0716) (width 0.25) (layer "F.Cu") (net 19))
 (segment (start 68.4915 83.0396) (end 68.6851 82.846) (width 0.25) (layer "F.Cu") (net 19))
 (segment (start 68.6851 82.846) (end 71.9205 82.846) (width 0.25) (layer "F.Cu") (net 19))
 (segment (start 86.0405 93.895) (end 86.0511 93.9056) (width 0.25) (layer "F.Cu") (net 21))
 (segment (start 86.0859 98.2208) (end 86.0859 97.705) (width 0.25) (layer "F.Cu") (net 21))
 (segment (start 86.0859 93.9404) (end 86.0511 93.9056) (width 0.25) (layer "F.Cu") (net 21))
 (segment (start 83.6915 93.895) (end 86.0405 93.895) (width 0.25) (layer "F.Cu") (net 21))
 (segment (start 84.1875 100.1192) (end 86.0859 98.2208) (width 0.25) (layer "F.Cu") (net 21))
 (segment (start 81.9003 97.832) (end 84.1875 100.1192) (width 0.25) (layer "F.Cu") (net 21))
 (segment (start 86.0859 97.705) (end 86.0859 93.9404) (width 0.25) (layer "F.Cu") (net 21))
 (segment (start 81.3945 97.832) (end 81.9003 97.832) (width 0.25) (layer "F.Cu") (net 21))
 (segment (start 90.3355 97.546) (end 90.3355 93.6984) (width 0.25) (layer "F.Cu") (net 7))
 (segment (start 90.3035 97.578) (end 90.3355 97.546) (width 0.25) (layer "F.Cu") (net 7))
 (segment (start 90.3035 97.578) (end 92.7485 97.578) (width 0.25) (layer "F.Cu") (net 7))
 (segment (start 94.2725 89.7614) (end 94.2725 85.513) (width 0.25) (layer "F.Cu") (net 7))
 (segment (start 90.3355 93.6984) (end 94.2725 89.7614) (width 0.25) (layer "F.Cu") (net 7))
 (segment (start 68.7801 92.911) (end 68.4915 93.1996) (width 0.25) (layer "F.Cu") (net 11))
 (segment (start 72.1745 94.211) (end 72.1745 93.133) (width 0.25) (layer "F.Cu") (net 11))
 (segment (start 65.8849 93.1996) (end 68.4915 93.1996) (width 0.25) (layer "F.Cu") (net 11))
 (segment (start 64.3005 94.784) (end 55.4105 94.784) (width 0.25) (layer "F.Cu") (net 11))
 (segment (start 64.3005 94.784) (end 65.8849 93.1996) (width 0.25) (layer "F.Cu") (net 11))
 (segment (start 72.1745 93.133) (end 71.9525 92.911) (width 0.25) (layer "F.Cu") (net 11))
 (segment (start 71.9525 92.911) (end 68.7801 92.911) (width 0.25) (layer "F.Cu") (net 11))
 (segment (start 70.9045 90.593) (end 70.9045 89.261) (width 0.25) (layer "F.Cu") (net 18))
 (segment (start 70.3015 91.196) (end 70.9045 90.593) (width 0.25) (layer "F.Cu") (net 18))
 (segment (start 68.4915 91.196) (end 70.3015 91.196) (width 0.25) (layer "F.Cu") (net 18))
 (segment (start 55.4105 89.704) (end 66.9995 89.704) (width 0.25) (layer "F.Cu") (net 18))
 (segment (start 66.9995 89.704) (end 68.4915 91.196) (width 0.25) (layer "F.Cu") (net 18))
 (segment (start 74.7145 86.402) (end 74.7145 89.261) (width 0.5) (layer "F.Cu") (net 2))
 (segment (start 63.2845 79.163) (end 65.6295 79.163) (width 0.5) (layer "F.Cu") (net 2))
 (segment (start 74.2065 80.56) (end 71.5504 80.56) (width 0.5) (layer "F.Cu") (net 2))
 (segment (start 70.1534 79.163) (end 70.9635 79.9731) (width 0.5) (layer "F.Cu") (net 2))
 (segment (start 71.5504 80.56) (end 70.9635 79.9731) (width 0.5) (layer "F.Cu") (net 2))
 (segment (start 65.6295 79.163) (end 70.1534 79.163) (width 0.5) (layer "F.Cu") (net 2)))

